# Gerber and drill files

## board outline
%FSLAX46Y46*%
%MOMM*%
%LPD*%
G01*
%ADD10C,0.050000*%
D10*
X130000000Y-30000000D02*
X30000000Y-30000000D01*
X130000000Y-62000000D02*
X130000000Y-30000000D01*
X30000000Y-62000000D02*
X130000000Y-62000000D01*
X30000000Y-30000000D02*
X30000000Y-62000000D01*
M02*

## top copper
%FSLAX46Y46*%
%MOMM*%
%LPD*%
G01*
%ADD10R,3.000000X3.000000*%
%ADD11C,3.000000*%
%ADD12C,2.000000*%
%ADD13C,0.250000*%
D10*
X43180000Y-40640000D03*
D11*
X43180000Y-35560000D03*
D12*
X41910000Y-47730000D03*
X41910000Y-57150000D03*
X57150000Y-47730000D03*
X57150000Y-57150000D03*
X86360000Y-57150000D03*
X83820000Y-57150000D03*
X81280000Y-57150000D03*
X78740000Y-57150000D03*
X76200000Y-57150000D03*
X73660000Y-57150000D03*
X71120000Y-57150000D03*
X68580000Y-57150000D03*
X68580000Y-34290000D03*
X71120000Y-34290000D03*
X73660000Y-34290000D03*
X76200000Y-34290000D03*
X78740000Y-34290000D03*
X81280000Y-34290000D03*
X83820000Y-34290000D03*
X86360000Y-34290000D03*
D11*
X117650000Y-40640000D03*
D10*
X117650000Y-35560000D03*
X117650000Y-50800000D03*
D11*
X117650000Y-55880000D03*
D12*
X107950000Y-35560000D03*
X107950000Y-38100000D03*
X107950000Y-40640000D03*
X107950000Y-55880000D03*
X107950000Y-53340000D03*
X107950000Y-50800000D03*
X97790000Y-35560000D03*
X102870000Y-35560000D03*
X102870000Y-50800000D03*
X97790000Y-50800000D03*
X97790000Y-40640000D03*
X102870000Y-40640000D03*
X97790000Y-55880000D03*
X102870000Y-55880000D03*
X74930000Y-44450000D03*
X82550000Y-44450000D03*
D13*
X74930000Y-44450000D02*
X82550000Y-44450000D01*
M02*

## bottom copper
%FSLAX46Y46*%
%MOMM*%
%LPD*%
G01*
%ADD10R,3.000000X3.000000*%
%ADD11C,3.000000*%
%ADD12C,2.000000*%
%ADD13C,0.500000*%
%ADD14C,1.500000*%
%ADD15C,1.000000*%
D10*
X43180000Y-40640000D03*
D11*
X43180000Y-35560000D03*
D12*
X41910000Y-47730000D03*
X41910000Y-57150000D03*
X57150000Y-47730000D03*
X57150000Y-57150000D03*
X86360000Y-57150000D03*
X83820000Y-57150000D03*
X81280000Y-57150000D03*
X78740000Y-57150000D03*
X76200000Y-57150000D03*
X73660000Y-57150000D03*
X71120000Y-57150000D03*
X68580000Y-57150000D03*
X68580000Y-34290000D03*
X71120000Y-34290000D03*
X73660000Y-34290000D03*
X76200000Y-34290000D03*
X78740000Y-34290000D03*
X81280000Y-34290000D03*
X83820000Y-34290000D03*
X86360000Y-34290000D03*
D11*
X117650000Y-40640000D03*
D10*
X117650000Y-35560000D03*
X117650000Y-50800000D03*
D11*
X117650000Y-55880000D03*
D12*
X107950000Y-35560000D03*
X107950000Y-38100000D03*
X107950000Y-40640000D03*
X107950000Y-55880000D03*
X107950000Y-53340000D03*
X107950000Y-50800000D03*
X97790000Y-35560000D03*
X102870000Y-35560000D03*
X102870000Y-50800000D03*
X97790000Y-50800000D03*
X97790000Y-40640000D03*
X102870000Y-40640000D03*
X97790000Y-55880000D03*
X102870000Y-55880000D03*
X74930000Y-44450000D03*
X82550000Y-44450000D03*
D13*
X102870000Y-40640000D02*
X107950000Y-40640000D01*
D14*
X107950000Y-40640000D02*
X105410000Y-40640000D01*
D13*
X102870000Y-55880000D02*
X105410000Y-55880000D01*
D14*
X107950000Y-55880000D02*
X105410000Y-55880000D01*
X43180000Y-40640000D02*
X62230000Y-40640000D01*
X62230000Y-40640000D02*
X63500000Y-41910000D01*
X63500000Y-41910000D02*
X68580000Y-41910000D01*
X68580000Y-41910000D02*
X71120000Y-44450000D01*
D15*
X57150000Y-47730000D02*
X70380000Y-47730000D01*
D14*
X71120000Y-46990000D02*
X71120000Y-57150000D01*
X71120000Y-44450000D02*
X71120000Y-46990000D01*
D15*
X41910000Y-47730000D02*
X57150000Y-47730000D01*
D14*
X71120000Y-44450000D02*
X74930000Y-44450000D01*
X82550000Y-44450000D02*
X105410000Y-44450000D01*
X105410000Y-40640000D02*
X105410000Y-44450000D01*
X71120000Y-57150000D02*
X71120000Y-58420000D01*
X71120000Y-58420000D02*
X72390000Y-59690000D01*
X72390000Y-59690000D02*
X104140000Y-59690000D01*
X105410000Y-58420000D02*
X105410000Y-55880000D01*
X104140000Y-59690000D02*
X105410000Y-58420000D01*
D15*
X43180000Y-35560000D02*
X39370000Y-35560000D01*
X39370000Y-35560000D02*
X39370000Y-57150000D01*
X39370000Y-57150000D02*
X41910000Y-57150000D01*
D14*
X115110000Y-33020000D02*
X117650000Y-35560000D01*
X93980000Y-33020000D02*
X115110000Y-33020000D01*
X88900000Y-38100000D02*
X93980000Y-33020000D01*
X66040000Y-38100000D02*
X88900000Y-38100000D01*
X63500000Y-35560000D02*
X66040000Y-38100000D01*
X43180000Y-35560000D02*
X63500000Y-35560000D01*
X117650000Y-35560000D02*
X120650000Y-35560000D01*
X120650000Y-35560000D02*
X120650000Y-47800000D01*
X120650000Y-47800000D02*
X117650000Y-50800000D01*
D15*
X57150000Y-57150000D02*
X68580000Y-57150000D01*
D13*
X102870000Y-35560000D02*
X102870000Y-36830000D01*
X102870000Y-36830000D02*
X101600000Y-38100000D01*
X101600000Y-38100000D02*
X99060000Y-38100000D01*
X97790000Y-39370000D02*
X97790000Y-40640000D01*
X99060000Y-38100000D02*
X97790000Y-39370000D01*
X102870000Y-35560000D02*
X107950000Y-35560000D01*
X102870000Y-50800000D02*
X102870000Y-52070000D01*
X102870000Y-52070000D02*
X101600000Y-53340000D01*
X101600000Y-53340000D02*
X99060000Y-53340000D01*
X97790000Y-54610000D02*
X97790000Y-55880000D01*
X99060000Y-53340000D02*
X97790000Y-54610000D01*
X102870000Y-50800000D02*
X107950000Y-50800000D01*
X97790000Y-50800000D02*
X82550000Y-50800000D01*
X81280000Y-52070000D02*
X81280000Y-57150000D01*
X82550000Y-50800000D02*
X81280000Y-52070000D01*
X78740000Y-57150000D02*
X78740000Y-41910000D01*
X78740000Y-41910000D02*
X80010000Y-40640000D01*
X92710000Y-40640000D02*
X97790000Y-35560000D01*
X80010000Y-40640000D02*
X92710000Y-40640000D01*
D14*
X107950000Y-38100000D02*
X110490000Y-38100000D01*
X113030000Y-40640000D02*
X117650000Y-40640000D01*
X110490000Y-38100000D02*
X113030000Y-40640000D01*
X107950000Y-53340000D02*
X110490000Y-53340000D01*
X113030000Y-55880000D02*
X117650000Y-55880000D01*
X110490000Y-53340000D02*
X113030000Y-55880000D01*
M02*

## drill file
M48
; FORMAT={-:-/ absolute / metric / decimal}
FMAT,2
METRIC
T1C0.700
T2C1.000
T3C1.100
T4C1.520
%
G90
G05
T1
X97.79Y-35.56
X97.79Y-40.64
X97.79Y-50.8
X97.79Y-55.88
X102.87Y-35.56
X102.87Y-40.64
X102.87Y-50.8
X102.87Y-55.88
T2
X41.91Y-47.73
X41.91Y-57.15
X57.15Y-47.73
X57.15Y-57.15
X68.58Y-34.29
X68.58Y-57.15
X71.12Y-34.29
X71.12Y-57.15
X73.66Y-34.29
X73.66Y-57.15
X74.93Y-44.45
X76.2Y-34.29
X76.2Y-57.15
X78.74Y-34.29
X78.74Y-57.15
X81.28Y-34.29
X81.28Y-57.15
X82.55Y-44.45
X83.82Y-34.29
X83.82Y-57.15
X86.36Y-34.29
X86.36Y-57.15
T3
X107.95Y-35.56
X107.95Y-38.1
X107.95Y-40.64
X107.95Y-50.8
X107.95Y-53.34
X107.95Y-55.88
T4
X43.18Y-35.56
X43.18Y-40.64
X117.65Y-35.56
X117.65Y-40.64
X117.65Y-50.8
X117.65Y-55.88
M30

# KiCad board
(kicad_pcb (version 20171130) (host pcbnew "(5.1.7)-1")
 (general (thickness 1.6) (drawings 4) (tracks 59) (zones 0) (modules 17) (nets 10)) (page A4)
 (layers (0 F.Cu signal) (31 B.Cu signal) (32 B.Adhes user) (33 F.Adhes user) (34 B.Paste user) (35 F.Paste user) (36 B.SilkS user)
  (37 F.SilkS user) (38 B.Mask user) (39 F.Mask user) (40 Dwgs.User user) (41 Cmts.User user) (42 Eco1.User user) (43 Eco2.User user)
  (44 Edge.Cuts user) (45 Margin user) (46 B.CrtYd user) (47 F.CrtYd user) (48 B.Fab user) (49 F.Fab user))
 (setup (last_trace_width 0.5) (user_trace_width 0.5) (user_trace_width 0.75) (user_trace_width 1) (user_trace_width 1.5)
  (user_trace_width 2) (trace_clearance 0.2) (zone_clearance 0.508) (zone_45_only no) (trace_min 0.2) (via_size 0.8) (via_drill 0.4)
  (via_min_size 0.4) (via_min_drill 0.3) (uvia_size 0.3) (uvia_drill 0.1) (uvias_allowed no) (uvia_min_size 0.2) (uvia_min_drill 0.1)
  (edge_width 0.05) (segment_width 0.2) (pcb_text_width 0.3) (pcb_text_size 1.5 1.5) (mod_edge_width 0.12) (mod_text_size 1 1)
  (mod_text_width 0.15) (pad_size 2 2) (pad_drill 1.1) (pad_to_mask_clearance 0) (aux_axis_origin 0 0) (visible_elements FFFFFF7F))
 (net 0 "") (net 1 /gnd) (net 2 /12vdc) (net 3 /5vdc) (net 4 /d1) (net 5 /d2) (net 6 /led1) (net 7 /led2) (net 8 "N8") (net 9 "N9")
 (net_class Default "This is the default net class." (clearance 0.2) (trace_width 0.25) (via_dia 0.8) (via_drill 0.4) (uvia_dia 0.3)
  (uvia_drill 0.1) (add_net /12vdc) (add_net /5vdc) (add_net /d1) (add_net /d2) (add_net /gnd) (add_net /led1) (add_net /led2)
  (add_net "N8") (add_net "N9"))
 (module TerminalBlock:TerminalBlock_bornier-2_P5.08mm (layer F.Cu) (at 43.18 40.64 90)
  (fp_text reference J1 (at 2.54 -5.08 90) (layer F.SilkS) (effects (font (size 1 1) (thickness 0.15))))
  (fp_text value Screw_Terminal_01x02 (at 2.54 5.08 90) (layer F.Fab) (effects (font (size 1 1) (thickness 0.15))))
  (pad 1 thru_hole rect (at 0 0 90) (size 3 3) (drill 1.52) (layers *.Cu *.Mask) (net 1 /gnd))
  (pad 2 thru_hole circle (at 5.08 0 90) (size 3 3) (drill 1.52) (layers *.Cu *.Mask) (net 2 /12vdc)))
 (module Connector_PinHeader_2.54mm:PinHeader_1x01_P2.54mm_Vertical (layer F.Cu) (at 41.91 47.73)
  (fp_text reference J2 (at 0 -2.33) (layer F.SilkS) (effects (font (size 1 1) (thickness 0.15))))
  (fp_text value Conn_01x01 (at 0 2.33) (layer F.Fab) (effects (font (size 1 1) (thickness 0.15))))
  (pad 1 thru_hole circle (at 0 0) (size 2 2) (drill 1) (layers *.Cu *.Mask) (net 1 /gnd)))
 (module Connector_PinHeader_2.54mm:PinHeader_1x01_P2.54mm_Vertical (layer F.Cu) (at 41.91 57.15)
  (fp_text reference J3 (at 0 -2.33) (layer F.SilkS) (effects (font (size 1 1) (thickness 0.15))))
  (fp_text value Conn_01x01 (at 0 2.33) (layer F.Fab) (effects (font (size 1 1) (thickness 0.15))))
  (pad 1 thru_hole circle (at 0 0) (size 2 2) (drill 1) (layers *.Cu *.Mask) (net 2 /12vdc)))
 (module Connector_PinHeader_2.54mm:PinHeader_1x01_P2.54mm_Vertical (layer F.Cu) (at 57.15 47.73)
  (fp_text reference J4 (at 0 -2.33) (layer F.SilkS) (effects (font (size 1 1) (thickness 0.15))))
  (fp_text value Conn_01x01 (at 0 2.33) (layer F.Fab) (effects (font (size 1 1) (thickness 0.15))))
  (pad 1 thru_hole circle (at 0 0) (size 2 2) (drill 1) (layers *.Cu *.Mask) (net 1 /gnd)))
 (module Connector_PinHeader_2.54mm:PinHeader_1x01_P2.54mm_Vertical (layer F.Cu) (at 57.15 57.15)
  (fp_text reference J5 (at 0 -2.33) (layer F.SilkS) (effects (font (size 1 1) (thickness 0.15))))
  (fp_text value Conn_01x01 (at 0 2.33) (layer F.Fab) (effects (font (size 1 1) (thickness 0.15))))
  (pad 1 thru_hole circle (at 0 0) (size 2 2) (drill 1) (layers *.Cu *.Mask) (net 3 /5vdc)))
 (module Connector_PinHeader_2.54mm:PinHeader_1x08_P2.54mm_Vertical (layer F.Cu) (at 68.58 57.15 90)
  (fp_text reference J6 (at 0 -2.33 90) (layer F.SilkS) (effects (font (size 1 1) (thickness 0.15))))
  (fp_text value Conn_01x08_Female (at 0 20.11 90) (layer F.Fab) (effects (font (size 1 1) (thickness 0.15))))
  (pad 8 thru_hole circle (at 0 17.78 90) (size 2 2) (drill 1) (layers *.Cu *.Mask))
  (pad 7 thru_hole circle (at 0 15.24 90) (size 2 2) (drill 1) (layers *.Cu *.Mask))
  (pad 6 thru_hole circle (at 0 12.7 90) (size 2 2) (drill 1) (layers *.Cu *.Mask) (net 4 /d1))
  (pad 5 thru_hole circle (at 0 10.16 90) (size 2 2) (drill 1) (layers *.Cu *.Mask) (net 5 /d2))
  (pad 4 thru_hole circle (at 0 7.62 90) (size 2 2) (drill 1) (layers *.Cu *.Mask))
  (pad 3 thru_hole circle (at 0 5.08 90) (size 2 2) (drill 1) (layers *.Cu *.Mask))
  (pad 2 thru_hole circle (at 0 2.54 90) (size 2 2) (drill 1) (layers *.Cu *.Mask) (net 1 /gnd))
  (pad 1 thru_hole circle (at 0 0 90) (size 2 2) (drill 1) (layers *.Cu *.Mask) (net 3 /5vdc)))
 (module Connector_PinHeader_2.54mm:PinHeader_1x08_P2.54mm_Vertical (layer F.Cu) (at 68.58 34.29 90)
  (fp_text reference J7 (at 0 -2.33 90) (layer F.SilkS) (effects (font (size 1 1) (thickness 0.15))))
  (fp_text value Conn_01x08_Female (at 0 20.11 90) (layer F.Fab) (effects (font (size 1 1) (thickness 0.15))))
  (pad 1 thru_hole circle (at 0 0 90) (size 2 2) (drill 1) (layers *.Cu *.Mask))
  (pad 2 thru_hole circle (at 0 2.54 90) (size 2 2) (drill 1) (layers *.Cu *.Mask))
  (pad 3 thru_hole circle (at 0 5.08 90) (size 2 2) (drill 1) (layers *.Cu *.Mask))
  (pad 4 thru_hole circle (at 0 7.62 90) (size 2 2) (drill 1) (layers *.Cu *.Mask))
  (pad 5 thru_hole circle (at 0 10.16 90) (size 2 2) (drill 1) (layers *.Cu *.Mask))
  (pad 6 thru_hole circle (at 0 12.7 90) (size 2 2) (drill 1) (layers *.Cu *.Mask))
  (pad 7 thru_hole circle (at 0 15.24 90) (size 2 2) (drill 1) (layers *.Cu *.Mask))
  (pad 8 thru_hole circle (at 0 17.78 90) (size 2 2) (drill 1) (layers *.Cu *.Mask)))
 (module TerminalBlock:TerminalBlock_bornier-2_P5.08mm (layer F.Cu) (at 117.65 35.56 270)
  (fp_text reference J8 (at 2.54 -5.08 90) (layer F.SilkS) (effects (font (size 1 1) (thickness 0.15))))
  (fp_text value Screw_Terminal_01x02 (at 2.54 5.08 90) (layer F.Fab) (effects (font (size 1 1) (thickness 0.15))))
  (pad 2 thru_hole circle (at 5.08 0 270) (size 3 3) (drill 1.52) (layers *.Cu *.Mask) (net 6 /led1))
  (pad 1 thru_hole rect (at 0 0 270) (size 3 3) (drill 1.52) (layers *.Cu *.Mask) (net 2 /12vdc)))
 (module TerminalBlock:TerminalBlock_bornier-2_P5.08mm (layer F.Cu) (at 117.65 50.8 270)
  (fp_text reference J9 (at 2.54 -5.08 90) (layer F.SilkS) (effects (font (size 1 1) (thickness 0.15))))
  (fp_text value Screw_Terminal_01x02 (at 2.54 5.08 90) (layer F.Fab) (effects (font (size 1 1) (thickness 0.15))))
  (pad 1 thru_hole rect (at 0 0 270) (size 3 3) (drill 1.52) (layers *.Cu *.Mask) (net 2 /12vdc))
  (pad 2 thru_hole circle (at 5.08 0 270) (size 3 3) (drill 1.52) (layers *.Cu *.Mask) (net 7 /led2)))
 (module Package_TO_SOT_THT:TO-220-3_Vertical (layer F.Cu) (at 107.95 35.56 270)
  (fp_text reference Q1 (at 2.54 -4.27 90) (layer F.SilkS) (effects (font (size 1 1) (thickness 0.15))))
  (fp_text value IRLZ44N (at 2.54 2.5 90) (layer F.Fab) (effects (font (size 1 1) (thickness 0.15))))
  (pad 1 thru_hole circle (at 0 0 270) (size 2 2) (drill 1.1) (layers *.Cu *.Mask) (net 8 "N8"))
  (pad 2 thru_hole circle (at 2.54 0 270) (size 2 2) (drill 1.1) (layers *.Cu *.Mask) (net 6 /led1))
  (pad 3 thru_hole circle (at 5.08 0 270) (size 2 2) (drill 1.1) (layers *.Cu *.Mask) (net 1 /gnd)))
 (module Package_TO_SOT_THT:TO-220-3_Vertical (layer F.Cu) (at 107.95 50.8 270)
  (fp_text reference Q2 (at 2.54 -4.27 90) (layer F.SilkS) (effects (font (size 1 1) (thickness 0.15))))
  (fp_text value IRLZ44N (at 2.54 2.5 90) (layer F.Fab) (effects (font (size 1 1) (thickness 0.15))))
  (pad 3 thru_hole circle (at 5.08 0 270) (size 2 2) (drill 1.1) (layers *.Cu *.Mask) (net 1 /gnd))
  (pad 2 thru_hole circle (at 2.54 0 270) (size 2 2) (drill 1.1) (layers *.Cu *.Mask) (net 7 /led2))
  (pad 1 thru_hole circle (at 0 0 270) (size 2 2) (drill 1.1) (layers *.Cu *.Mask) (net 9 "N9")))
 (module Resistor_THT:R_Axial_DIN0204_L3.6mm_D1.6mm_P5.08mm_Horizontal (layer F.Cu) (at 102.87 35.56 180)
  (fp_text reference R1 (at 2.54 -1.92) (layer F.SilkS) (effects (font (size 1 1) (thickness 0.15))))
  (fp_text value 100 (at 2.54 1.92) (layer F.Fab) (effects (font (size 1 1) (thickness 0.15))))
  (pad 2 thru_hole circle (at 5.08 0 180) (size 2 2) (drill 0.7) (layers *.Cu *.Mask) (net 5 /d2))
  (pad 1 thru_hole circle (at 0 0 180) (size 2 2) (drill 0.7) (layers *.Cu *.Mask) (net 8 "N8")))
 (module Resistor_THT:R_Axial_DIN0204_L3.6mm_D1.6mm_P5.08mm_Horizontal (layer F.Cu) (at 97.79 50.8)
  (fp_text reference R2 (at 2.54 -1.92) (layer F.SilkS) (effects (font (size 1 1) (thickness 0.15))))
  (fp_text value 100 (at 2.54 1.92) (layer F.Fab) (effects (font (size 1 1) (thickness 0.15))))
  (pad 2 thru_hole circle (at 5.08 0) (size 2 2) (drill 0.7) (layers *.Cu *.Mask) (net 9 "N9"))
  (pad 1 thru_hole circle (at 0 0) (size 2 2) (drill 0.7) (layers *.Cu *.Mask) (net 4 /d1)))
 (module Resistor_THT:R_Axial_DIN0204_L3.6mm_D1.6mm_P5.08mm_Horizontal (layer F.Cu) (at 97.79 40.64)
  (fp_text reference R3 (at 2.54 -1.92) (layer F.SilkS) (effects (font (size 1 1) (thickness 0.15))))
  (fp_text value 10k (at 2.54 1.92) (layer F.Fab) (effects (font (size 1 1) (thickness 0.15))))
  (pad 1 thru_hole circle (at 0 0) (size 2 2) (drill 0.7) (layers *.Cu *.Mask) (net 8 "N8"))
  (pad 2 thru_hole circle (at 5.08 0) (size 2 2) (drill 0.7) (layers *.Cu *.Mask) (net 1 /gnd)))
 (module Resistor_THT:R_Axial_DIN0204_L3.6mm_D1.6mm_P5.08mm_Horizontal (layer F.Cu) (at 97.79 55.88)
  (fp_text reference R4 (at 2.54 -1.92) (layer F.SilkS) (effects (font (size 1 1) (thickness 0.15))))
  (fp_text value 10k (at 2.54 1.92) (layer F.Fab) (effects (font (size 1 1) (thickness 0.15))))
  (pad 1 thru_hole circle (at 0 0) (size 2 2) (drill 0.7) (layers *.Cu *.Mask) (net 9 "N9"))
  (pad 2 thru_hole circle (at 5.08 0) (size 2 2) (drill 0.7) (layers *.Cu *.Mask) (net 1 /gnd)))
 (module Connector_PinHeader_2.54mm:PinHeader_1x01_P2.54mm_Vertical (layer F.Cu) (at 74.93 44.45)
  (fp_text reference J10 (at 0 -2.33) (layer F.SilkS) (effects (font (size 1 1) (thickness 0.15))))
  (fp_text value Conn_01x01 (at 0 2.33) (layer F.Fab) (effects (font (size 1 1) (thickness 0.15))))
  (pad 1 thru_hole circle (at 0 0) (size 2 2) (drill 1) (layers *.Cu *.Mask) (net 1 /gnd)))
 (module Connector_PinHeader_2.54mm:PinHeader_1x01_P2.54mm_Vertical (layer F.Cu) (at 82.55 44.45)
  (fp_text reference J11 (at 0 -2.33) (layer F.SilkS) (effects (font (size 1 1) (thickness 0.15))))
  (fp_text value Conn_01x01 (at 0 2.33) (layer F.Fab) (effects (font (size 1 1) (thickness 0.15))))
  (pad 1 thru_hole circle (at 0 0) (size 2 2) (drill 1) (layers *.Cu *.Mask) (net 1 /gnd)))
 (gr_line (start 130 30) (end 30 30) (layer Edge.Cuts) (width 0.05))
 (gr_line (start 130 62) (end 130 30) (layer Edge.Cuts) (width 0.05))
 (gr_line (start 30 62) (end 130 62) (layer Edge.Cuts) (width 0.05))
 (gr_line (start 30 30) (end 30 62) (layer Edge.Cuts) (width 0.05))
 (segment (start 102.87 40.64) (end 107.95 40.64) (width 0.5) (layer B.Cu) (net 1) (status 30))
 (segment (start 107.95 40.64) (end 105.41 40.64) (width 1.5) (layer B.Cu) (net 1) (status 10))
 (segment (start 102.87 55.88) (end 105.41 55.88) (width 0.5) (layer B.Cu) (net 1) (status 10))
 (segment (start 107.95 55.88) (end 105.41 55.88) (width 1.5) (layer B.Cu) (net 1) (status 10))
 (segment (start 43.18 40.64) (end 62.23 40.64) (width 1.5) (layer B.Cu) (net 1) (status 10))
 (segment (start 62.23 40.64) (end 63.5 41.91) (width 1.5) (layer B.Cu) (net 1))
 (segment (start 63.5 41.91) (end 68.58 41.91) (width 1.5) (layer B.Cu) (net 1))
 (segment (start 68.58 41.91) (end 71.12 44.45) (width 1.5) (layer B.Cu) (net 1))
 (segment (start 57.15 47.73) (end 70.38 47.73) (width 1) (layer B.Cu) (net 1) (status 10))
 (segment (start 71.12 46.99) (end 71.12 57.15) (width 1.5) (layer B.Cu) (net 1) (status 1000020))
 (segment (start 71.12 44.45) (end 71.12 46.99) (width 1.5) (layer B.Cu) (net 1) (status 1000000))
 (segment (start 41.91 47.73) (end 57.15 47.73) (width 1) (layer B.Cu) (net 1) (status 30))
 (segment (start 71.12 44.45) (end 74.93 44.45) (width 1.5) (layer B.Cu) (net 1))
 (segment (start 82.55 44.45) (end 105.41 44.45) (width 1.5) (layer B.Cu) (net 1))
 (segment (start 105.41 40.64) (end 105.41 44.45) (width 1.5) (layer B.Cu) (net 1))
 (segment (start 74.93 44.45) (end 82.55 44.45) (width 0.25) (layer F.Cu) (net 1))
 (segment (start 71.12 57.15) (end 71.12 58.42) (width 1.5) (layer B.Cu) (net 1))
 (segment (start 71.12 58.42) (end 72.39 59.69) (width 1.5) (layer B.Cu) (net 1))
 (segment (start 72.39 59.69) (end 104.14 59.69) (width 1.5) (layer B.Cu) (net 1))
 (segment (start 105.41 58.42) (end 105.41 55.88) (width 1.5) (layer B.Cu) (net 1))
 (segment (start 104.14 59.69) (end 105.41 58.42) (width 1.5) (layer B.Cu) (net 1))
 (segment (start 43.18 35.56) (end 39.37 35.56) (width 1) (layer B.Cu) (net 2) (status 10))
 (segment (start 39.37 35.56) (end 39.37 57.15) (width 1) (layer B.Cu) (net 2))
 (segment (start 39.37 57.15) (end 41.91 57.15) (width 1) (layer B.Cu) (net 2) (status 20))
 (segment (start 115.11 33.02) (end 117.65 35.56) (width 1.5) (layer B.Cu) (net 2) (status 20))
 (segment (start 93.98 33.02) (end 115.11 33.02) (width 1.5) (layer B.Cu) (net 2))
 (segment (start 88.9 38.1) (end 93.98 33.02) (width 1.5) (layer B.Cu) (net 2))
 (segment (start 66.04 38.1) (end 88.9 38.1) (width 1.5) (layer B.Cu) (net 2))
 (segment (start 63.5 35.56) (end 66.04 38.1) (width 1.5) (layer B.Cu) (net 2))
 (segment (start 43.18 35.56) (end 63.5 35.56) (width 1.5) (layer B.Cu) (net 2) (status 10))
 (segment (start 117.65 35.56) (end 120.65 35.56) (width 1.5) (layer B.Cu) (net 2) (status 10))
 (segment (start 120.65 35.56) (end 120.65 47.8) (width 1.5) (layer B.Cu) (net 2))
 (segment (start 120.65 47.8) (end 117.65 50.8) (width 1.5) (layer B.Cu) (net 2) (status 20))
 (segment (start 57.15 57.15) (end 68.58 57.15) (width 1) (layer B.Cu) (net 3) (status 30))
 (segment (start 102.87 35.56) (end 102.87 36.83) (width 0.5) (layer B.Cu) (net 8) (status 10))
 (segment (start 102.87 36.83) (end 101.6 38.1) (width 0.5) (layer B.Cu) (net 8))
 (segment (start 101.6 38.1) (end 99.06 38.1) (width 0.5) (layer B.Cu) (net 8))
 (segment (start 97.79 39.37) (end 97.79 40.64) (width 0.5) (layer B.Cu) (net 8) (status 20))
 (segment (start 99.06 38.1) (end 97.79 39.37) (width 0.5) (layer B.Cu) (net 8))
 (segment (start 102.87 35.56) (end 107.95 35.56) (width 0.5) (layer B.Cu) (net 8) (status 30))
 (segment (start 102.87 50.8) (end 102.87 52.07) (width 0.5) (layer B.Cu) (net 9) (status 10))
 (segment (start 102.87 52.07) (end 101.6 53.34) (width 0.5) (layer B.Cu) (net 9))
 (segment (start 101.6 53.34) (end 99.06 53.34) (width 0.5) (layer B.Cu) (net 9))
 (segment (start 97.79 54.61) (end 97.79 55.88) (width 0.5) (layer B.Cu) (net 9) (status 20))
 (segment (start 99.06 53.34) (end 97.79 54.61) (width 0.5) (layer B.Cu) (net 9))
 (segment (start 102.87 50.8) (end 107.95 50.8) (width 0.5) (layer B.Cu) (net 9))
 (segment (start 97.79 50.8) (end 82.55 50.8) (width 0.5) (layer B.Cu) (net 4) (status 10))
 (segment (start 81.28 52.07) (end 81.28 57.15) (width 0.5) (layer B.Cu) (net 4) (status 20))
 (segment (start 82.55 50.8) (end 81.28 52.07) (width 0.5) (layer B.Cu) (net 4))
 (segment (start 78.74 57.15) (end 78.74 41.91) (width 0.5) (layer B.Cu) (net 5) (status 10))
 (segment (start 78.74 41.91) (end 80.01 40.64) (width 0.5) (layer B.Cu) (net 5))
 (segment (start 92.71 40.64) (end 97.79 35.56) (width 0.5) (layer B.Cu) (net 5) (status 20))
 (segment (start 80.01 40.64) (end 92.71 40.64) (width 0.5) (layer B.Cu) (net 5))
 (segment (start 107.95 38.1) (end 110.49 38.1) (width 1.5) (layer B.Cu) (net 6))
 (segment (start 113.03 40.64) (end 117.65 40.64) (width 1.5) (layer B.Cu) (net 6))
 (segment (start 110.49 38.1) (end 113.03 40.64) (width 1.5) (layer B.Cu) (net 6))
 (segment (start 107.95 53.34) (end 110.49 53.34) (width 1.5) (layer B.Cu) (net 7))
 (segment (start 113.03 55.88) (end 117.65 55.88) (width 1.5) (layer B.Cu) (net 7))
 (segment (start 110.49 53.34) (end 113.03 55.88) (width 1.5) (layer B.Cu) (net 7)))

